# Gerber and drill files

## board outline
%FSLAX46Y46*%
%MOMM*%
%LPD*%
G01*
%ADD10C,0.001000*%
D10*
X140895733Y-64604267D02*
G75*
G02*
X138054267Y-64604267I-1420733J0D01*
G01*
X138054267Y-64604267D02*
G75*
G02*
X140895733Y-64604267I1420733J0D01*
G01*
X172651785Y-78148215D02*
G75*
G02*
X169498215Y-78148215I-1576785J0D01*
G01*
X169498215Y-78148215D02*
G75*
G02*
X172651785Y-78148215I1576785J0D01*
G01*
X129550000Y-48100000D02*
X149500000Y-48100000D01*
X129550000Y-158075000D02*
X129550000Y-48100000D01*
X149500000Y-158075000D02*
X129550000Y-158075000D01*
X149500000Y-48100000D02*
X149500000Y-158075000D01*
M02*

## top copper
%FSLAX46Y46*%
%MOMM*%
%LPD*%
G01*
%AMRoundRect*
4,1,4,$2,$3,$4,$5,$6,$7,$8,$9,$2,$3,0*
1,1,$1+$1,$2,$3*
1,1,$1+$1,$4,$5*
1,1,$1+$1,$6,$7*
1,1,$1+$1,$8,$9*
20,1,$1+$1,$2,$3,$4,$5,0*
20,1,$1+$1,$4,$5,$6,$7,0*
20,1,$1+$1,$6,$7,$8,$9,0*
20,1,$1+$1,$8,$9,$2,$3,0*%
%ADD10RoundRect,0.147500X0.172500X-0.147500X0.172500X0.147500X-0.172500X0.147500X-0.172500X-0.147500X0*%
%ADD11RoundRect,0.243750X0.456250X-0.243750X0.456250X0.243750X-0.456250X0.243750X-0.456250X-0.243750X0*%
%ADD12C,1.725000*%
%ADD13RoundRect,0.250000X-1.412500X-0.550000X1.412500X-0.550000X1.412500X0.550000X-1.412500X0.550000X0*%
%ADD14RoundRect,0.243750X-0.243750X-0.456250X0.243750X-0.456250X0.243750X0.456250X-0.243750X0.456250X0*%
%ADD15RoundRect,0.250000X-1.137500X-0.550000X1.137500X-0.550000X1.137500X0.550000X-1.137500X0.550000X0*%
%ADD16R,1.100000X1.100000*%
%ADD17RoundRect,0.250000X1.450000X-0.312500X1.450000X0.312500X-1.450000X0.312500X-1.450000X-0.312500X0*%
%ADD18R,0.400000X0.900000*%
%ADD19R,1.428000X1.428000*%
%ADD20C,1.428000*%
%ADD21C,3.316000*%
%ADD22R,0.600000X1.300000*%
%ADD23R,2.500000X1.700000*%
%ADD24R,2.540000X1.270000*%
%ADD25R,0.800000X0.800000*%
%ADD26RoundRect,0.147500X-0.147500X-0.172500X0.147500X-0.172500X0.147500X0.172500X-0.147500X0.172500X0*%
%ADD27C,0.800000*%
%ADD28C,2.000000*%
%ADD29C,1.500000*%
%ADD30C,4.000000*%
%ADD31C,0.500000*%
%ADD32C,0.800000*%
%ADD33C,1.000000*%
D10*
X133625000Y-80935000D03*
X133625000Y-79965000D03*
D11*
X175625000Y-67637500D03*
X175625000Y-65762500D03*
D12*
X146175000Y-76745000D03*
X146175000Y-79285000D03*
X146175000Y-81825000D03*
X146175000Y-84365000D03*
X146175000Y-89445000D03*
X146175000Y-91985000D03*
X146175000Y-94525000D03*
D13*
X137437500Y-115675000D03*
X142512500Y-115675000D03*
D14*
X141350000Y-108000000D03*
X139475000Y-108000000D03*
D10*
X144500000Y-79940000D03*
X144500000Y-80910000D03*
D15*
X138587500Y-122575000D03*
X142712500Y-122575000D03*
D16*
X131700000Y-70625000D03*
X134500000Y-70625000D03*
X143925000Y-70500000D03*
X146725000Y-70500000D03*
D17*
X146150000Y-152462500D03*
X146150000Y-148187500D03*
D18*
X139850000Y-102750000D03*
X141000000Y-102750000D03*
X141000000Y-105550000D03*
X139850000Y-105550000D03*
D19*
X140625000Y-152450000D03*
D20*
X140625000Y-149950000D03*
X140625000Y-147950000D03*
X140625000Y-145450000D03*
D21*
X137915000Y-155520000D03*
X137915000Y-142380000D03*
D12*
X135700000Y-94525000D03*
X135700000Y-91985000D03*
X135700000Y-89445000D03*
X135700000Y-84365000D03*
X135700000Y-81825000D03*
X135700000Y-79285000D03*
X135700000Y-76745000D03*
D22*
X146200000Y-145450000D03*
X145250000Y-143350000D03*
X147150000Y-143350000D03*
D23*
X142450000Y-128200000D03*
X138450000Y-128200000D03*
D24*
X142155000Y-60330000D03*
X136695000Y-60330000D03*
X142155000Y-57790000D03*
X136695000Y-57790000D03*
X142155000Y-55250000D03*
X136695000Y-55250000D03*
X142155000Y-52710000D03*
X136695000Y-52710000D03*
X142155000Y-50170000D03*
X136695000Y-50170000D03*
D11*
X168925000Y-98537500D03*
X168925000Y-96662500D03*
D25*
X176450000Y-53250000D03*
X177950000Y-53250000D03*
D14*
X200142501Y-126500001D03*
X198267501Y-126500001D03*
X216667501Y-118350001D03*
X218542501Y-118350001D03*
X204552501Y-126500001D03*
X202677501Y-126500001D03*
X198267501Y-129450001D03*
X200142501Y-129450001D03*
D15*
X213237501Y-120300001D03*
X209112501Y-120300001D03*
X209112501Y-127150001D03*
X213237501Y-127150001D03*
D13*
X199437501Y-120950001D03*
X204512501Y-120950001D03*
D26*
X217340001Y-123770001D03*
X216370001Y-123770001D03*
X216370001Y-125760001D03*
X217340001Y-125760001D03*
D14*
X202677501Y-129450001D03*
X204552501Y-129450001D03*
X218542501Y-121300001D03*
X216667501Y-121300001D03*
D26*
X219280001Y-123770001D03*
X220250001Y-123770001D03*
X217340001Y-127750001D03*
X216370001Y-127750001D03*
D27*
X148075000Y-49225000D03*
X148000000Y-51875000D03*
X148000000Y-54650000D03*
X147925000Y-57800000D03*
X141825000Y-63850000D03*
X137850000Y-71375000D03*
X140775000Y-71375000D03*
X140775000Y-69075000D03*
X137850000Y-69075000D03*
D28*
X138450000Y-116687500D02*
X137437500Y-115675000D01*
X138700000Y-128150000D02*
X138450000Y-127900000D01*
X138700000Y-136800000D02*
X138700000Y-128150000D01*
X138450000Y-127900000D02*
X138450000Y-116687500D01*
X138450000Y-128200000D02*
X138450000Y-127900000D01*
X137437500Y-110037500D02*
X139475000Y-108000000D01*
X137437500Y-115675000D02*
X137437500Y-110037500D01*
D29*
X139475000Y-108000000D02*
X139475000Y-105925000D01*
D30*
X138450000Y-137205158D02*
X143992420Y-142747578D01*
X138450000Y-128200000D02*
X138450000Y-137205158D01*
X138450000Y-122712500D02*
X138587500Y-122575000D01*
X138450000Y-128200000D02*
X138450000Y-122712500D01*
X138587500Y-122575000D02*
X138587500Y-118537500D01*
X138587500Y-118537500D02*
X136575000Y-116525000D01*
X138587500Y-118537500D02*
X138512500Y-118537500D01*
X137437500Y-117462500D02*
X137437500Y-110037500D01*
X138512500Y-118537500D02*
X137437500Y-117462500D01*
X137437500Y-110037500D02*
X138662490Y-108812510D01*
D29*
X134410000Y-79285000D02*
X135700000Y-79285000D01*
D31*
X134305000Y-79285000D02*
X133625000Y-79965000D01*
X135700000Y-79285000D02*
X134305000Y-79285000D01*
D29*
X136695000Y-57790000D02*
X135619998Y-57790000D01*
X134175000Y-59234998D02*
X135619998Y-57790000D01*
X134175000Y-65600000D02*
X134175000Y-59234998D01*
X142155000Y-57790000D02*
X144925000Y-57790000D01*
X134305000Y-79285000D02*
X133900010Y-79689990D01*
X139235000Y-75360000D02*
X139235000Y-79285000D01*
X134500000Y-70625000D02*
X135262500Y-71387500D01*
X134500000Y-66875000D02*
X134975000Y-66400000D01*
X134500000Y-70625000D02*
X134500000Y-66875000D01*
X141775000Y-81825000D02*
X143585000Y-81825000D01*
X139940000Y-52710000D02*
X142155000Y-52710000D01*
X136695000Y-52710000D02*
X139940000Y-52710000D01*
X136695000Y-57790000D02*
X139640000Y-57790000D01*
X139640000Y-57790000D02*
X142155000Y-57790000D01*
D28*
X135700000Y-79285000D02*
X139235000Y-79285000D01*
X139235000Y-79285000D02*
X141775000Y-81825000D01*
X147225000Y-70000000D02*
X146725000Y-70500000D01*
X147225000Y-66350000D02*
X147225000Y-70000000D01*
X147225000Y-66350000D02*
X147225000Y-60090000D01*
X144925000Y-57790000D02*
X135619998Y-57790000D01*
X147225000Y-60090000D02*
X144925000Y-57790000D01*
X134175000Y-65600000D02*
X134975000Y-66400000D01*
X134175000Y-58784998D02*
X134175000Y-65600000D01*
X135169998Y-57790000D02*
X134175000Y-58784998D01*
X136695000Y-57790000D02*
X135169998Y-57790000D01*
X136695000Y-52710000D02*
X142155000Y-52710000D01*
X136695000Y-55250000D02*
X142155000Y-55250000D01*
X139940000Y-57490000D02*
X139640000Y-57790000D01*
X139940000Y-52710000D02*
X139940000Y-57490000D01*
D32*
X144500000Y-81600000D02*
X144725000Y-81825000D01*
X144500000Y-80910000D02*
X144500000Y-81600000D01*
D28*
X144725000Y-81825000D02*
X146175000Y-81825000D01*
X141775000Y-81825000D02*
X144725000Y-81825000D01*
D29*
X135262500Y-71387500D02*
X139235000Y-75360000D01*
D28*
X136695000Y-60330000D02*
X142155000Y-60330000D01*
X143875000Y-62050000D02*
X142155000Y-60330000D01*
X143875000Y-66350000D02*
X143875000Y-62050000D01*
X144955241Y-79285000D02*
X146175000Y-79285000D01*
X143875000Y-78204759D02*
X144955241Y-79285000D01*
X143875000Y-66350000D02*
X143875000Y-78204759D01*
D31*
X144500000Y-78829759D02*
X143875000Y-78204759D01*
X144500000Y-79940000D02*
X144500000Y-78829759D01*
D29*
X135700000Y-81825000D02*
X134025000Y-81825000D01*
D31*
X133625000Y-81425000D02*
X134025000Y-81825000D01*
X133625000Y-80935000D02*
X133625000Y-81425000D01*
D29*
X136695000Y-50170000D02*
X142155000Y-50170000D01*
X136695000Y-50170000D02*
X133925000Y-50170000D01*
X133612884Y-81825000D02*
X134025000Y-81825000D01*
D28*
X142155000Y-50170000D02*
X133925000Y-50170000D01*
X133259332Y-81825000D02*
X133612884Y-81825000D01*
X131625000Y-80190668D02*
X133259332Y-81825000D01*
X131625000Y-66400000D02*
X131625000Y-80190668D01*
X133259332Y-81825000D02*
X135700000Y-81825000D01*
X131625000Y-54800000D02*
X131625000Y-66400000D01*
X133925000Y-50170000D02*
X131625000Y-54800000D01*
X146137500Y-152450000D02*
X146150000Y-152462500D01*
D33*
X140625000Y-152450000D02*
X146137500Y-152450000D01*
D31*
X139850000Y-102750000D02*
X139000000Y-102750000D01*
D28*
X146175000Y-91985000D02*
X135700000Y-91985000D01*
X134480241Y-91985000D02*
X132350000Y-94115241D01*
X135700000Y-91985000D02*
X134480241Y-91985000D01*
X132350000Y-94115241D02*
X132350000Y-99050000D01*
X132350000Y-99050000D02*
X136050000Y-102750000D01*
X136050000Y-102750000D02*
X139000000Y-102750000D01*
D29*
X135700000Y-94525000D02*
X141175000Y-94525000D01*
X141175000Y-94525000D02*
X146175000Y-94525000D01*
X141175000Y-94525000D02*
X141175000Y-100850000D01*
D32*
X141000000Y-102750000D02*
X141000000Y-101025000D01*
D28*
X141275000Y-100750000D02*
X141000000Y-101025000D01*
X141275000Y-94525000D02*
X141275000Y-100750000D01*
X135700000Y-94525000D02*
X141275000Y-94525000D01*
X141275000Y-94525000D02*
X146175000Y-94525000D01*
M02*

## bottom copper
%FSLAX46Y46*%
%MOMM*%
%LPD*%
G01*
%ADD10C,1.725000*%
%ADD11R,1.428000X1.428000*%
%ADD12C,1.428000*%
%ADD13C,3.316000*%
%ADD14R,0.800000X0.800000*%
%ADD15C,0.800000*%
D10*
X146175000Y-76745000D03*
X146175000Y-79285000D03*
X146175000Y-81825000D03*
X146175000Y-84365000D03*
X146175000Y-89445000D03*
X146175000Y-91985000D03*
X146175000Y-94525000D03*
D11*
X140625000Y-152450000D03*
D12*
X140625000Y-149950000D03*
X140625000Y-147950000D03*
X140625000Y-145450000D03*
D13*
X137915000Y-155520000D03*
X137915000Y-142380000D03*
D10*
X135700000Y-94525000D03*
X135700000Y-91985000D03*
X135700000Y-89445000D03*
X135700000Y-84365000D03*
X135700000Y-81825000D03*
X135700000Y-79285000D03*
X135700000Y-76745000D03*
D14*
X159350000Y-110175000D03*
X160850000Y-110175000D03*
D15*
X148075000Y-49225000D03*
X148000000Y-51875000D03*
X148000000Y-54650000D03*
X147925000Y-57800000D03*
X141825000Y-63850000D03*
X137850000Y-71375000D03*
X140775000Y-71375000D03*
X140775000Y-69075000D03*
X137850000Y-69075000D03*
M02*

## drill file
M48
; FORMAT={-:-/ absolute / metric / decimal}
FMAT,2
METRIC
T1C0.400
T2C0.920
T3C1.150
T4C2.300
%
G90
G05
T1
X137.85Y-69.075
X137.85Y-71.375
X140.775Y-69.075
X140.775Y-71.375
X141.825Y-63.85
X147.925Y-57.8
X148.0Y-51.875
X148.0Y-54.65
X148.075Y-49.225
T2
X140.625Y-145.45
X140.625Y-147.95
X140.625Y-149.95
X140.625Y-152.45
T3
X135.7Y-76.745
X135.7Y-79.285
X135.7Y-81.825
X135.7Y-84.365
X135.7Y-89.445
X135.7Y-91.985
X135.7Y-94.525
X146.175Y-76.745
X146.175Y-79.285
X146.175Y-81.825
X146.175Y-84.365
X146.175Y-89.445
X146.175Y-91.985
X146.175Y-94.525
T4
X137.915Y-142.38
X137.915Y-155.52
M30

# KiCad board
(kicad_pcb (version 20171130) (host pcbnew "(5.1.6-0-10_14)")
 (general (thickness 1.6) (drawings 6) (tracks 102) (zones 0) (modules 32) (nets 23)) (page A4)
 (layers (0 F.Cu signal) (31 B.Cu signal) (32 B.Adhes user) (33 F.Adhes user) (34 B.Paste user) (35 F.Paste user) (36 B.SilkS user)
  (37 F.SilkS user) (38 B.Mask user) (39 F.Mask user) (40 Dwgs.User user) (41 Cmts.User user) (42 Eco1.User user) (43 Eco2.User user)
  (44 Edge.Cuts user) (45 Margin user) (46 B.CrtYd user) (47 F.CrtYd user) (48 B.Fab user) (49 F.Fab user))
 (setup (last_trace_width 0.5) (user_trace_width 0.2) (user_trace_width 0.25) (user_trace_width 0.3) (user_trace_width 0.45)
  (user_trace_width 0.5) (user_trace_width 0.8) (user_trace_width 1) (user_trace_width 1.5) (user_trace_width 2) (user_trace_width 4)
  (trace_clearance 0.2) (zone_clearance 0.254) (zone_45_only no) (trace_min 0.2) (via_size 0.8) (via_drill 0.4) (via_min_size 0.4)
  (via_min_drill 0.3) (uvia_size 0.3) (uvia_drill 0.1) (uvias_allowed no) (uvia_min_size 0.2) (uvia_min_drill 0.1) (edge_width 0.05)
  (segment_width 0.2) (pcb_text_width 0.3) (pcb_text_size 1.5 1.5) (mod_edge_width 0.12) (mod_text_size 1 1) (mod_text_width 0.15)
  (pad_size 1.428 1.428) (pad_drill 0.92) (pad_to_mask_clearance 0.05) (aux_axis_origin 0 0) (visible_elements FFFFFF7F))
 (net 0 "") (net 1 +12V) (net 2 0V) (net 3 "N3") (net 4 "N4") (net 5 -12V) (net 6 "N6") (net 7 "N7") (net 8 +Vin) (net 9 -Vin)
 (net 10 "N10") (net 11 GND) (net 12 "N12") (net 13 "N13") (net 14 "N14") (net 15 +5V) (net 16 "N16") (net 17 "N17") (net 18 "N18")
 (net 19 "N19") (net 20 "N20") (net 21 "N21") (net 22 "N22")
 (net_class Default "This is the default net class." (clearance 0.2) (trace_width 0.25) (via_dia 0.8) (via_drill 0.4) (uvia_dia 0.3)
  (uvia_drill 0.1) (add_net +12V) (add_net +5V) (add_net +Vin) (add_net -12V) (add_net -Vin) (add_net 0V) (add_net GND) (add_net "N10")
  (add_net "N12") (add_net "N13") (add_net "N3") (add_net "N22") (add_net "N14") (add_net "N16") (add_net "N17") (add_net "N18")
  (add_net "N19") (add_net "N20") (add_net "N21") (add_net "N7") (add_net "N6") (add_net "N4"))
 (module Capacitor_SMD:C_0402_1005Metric (layer F.Cu) (at 133.625 80.45 90)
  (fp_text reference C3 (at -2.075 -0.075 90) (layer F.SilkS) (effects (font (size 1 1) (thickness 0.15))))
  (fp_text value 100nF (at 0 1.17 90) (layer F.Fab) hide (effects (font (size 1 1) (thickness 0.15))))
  (pad 1 smd roundrect (at -0.485 0 90) (size 0.59 0.64) (layers F.Cu F.Paste F.Mask) (roundrect_rratio 0.25) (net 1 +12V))
  (pad 2 smd roundrect (at 0.485 0 90) (size 0.59 0.64) (layers F.Cu F.Paste F.Mask) (roundrect_rratio 0.25) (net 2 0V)))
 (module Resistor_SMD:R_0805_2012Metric (layer F.Cu) (at 175.625 66.7 90)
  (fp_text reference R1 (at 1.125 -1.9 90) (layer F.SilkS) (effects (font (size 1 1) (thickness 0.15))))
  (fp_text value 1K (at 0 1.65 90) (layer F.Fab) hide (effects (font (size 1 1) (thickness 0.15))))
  (pad 1 smd roundrect (at -0.9375 0 90) (size 0.975 1.4) (layers F.Cu F.Paste F.Mask) (roundrect_rratio 0.25) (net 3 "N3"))
  (pad 2 smd roundrect (at 0.9375 0 90) (size 0.975 1.4) (layers F.Cu F.Paste F.Mask) (roundrect_rratio 0.25) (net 2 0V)))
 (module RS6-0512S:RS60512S (layer B.Cu) (at 146.175 94.525 90)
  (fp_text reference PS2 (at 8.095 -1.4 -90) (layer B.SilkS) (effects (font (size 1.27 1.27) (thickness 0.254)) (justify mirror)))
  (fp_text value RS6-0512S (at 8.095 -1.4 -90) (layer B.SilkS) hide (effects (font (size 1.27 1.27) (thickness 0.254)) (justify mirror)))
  (pad 8 thru_hole circle (at 17.78 0) (size 1.725 1.725) (drill 1.15) (layers *.Cu *.Mask B.SilkS) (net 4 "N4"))
  (pad 7 thru_hole circle (at 15.24 0) (size 1.725 1.725) (drill 1.15) (layers *.Cu *.Mask B.SilkS) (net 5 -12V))
  (pad 6 thru_hole circle (at 12.7 0) (size 1.725 1.725) (drill 1.15) (layers *.Cu *.Mask B.SilkS) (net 2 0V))
  (pad 5 thru_hole circle (at 10.16 0) (size 1.725 1.725) (drill 1.15) (layers *.Cu *.Mask B.SilkS) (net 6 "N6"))
  (pad 3 thru_hole circle (at 5.08 0) (size 1.725 1.725) (drill 1.15) (layers *.Cu *.Mask B.SilkS) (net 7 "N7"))
  (pad 2 thru_hole circle (at 2.54 0) (size 1.725 1.725) (drill 1.15) (layers *.Cu *.Mask B.SilkS) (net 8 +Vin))
  (pad 1 thru_hole circle (at 0 0) (size 1.725 1.725) (drill 1.15) (layers *.Cu *.Mask B.SilkS) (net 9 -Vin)))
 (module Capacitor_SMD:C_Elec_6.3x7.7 (layer F.Cu) (at 139.975 115.675)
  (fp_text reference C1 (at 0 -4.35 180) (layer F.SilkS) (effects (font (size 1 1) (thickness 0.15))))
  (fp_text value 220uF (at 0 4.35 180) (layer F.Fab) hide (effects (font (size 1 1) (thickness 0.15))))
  (pad 1 smd roundrect (at -2.5375 0) (size 3.325 1.6) (layers F.Cu F.Paste F.Mask) (roundrect_rratio 0.15625) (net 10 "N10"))
  (pad 2 smd roundrect (at 2.5375 0) (size 3.325 1.6) (layers F.Cu F.Paste F.Mask) (roundrect_rratio 0.15625) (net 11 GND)))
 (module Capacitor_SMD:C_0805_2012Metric (layer F.Cu) (at 140.4125 108)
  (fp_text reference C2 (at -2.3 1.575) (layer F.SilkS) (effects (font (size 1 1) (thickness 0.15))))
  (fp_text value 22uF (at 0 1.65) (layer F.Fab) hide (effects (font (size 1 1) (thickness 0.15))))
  (pad 2 smd roundrect (at 0.9375 0) (size 0.975 1.4) (layers F.Cu F.Paste F.Mask) (roundrect_rratio 0.25) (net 11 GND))
  (pad 1 smd roundrect (at -0.9375 0) (size 0.975 1.4) (layers F.Cu F.Paste F.Mask) (roundrect_rratio 0.25) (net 10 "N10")))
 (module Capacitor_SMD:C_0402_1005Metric (layer F.Cu) (at 144.5 80.425 90)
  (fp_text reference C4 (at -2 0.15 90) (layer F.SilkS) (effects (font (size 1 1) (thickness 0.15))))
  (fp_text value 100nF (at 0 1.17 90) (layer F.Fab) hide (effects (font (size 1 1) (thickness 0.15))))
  (pad 2 smd roundrect (at 0.485 0 90) (size 0.59 0.64) (layers F.Cu F.Paste F.Mask) (roundrect_rratio 0.25) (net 5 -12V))
  (pad 1 smd roundrect (at -0.485 0 90) (size 0.59 0.64) (layers F.Cu F.Paste F.Mask) (roundrect_rratio 0.25) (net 2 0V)))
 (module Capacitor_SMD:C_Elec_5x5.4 (layer F.Cu) (at 140.65 122.575)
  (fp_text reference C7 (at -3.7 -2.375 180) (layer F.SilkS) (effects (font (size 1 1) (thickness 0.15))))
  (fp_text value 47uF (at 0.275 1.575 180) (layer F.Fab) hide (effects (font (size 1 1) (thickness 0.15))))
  (pad 1 smd roundrect (at -2.0625 0) (size 2.775 1.6) (layers F.Cu F.Paste F.Mask) (roundrect_rratio 0.15625) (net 10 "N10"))
  (pad 2 smd roundrect (at 2.0625 0) (size 2.775 1.6) (layers F.Cu F.Paste F.Mask) (roundrect_rratio 0.15625) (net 11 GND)))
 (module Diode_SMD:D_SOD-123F (layer F.Cu) (at 133.1 70.625)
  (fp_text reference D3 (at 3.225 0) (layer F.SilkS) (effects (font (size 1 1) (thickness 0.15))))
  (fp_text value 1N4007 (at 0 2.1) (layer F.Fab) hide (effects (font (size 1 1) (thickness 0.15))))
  (pad 1 smd rect (at -1.4 0) (size 1.1 1.1) (layers F.Cu F.Paste F.Mask) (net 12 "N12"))
  (pad 2 smd rect (at 1.4 0) (size 1.1 1.1) (layers F.Cu F.Paste F.Mask) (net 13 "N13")))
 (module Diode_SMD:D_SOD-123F (layer F.Cu) (at 145.325 70.5 180)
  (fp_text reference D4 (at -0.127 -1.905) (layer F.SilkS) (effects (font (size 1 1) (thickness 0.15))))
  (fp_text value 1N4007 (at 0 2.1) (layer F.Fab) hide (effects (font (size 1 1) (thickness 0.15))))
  (pad 2 smd rect (at 1.4 0 180) (size 1.1 1.1) (layers F.Cu F.Paste F.Mask) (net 5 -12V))
  (pad 1 smd rect (at -1.4 0 180) (size 1.1 1.1) (layers F.Cu F.Paste F.Mask) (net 13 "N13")))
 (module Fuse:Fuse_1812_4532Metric (layer F.Cu) (at 146.15 150.325 90)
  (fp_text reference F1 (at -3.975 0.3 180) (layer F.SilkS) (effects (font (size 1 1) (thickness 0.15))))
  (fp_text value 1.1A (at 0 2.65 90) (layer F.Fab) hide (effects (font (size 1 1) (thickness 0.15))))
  (pad 1 smd roundrect (at -2.1375 0 90) (size 1.125 3.4) (layers F.Cu F.Paste F.Mask) (roundrect_rratio 0.222222) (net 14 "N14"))
  (pad 2 smd roundrect (at 2.1375 0 90) (size 1.125 3.4) (layers F.Cu F.Paste F.Mask) (roundrect_rratio 0.222222) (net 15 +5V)))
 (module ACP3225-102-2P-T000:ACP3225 (layer F.Cu) (at 140.425 104.15 90)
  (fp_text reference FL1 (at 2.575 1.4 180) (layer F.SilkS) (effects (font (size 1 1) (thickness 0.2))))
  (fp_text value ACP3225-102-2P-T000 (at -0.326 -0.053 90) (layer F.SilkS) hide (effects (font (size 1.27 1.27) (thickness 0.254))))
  (pad 4 smd rect (at 1.4 -0.575 180) (size 0.4 0.9) (layers F.Cu F.Paste F.Mask) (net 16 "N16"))
  (pad 3 smd rect (at 1.4 0.575 180) (size 0.4 0.9) (layers F.Cu F.Paste F.Mask) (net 9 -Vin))
  (pad 2 smd rect (at -1.4 0.575 180) (size 0.4 0.9) (layers F.Cu F.Paste F.Mask) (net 11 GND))
  (pad 1 smd rect (at -1.4 -0.575 180) (size 0.4 0.9) (layers F.Cu F.Paste F.Mask) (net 10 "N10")))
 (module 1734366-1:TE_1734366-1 (layer B.Cu) (at 140.625 152.45 90)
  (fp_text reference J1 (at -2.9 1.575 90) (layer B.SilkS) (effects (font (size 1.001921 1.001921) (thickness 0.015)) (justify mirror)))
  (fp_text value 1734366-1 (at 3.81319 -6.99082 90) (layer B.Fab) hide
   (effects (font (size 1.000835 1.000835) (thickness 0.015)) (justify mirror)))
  (pad 1 thru_hole rect (at 0 0 90) (size 1.428 1.428) (drill 0.92) (layers *.Cu *.Mask) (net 14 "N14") (zone_connect 1))
  (pad 2 thru_hole circle (at 2.5 0 90) (size 1.428 1.428) (drill 0.92) (layers *.Cu *.Mask) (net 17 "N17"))
  (pad 3 thru_hole circle (at 4.5 0 90) (size 1.428 1.428) (drill 0.92) (layers *.Cu *.Mask) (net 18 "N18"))
  (pad 4 thru_hole circle (at 7 0 90) (size 1.428 1.428) (drill 0.92) (layers *.Cu *.Mask) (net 11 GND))
  (pad SH1 thru_hole circle (at -3.07 -2.71 90) (size 3.316 3.316) (drill 2.3) (layers *.Cu *.Mask) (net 11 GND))
  (pad SH2 thru_hole circle (at 10.07 -2.71 90) (size 3.316 3.316) (drill 2.3) (layers *.Cu *.Mask) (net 11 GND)))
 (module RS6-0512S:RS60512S (layer B.Cu) (at 135.7 94.525 90)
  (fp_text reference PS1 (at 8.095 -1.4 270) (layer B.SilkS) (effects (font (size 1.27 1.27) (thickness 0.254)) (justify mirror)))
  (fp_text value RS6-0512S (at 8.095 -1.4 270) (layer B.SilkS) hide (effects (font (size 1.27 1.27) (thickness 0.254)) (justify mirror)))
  (pad 1 thru_hole circle (at 0 0) (size 1.725 1.725) (drill 1.15) (layers *.Cu *.Mask B.SilkS) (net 9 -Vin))
  (pad 2 thru_hole circle (at 2.54 0) (size 1.725 1.725) (drill 1.15) (layers *.Cu *.Mask B.SilkS) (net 8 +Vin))
  (pad 3 thru_hole circle (at 5.08 0) (size 1.725 1.725) (drill 1.15) (layers *.Cu *.Mask B.SilkS) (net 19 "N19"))
  (pad 5 thru_hole circle (at 10.16 0) (size 1.725 1.725) (drill 1.15) (layers *.Cu *.Mask B.SilkS) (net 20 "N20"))
  (pad 6 thru_hole circle (at 12.7 0) (size 1.725 1.725) (drill 1.15) (layers *.Cu *.Mask B.SilkS) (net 1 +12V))
  (pad 7 thru_hole circle (at 15.24 0) (size 1.725 1.725) (drill 1.15) (layers *.Cu *.Mask B.SilkS) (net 2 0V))
  (pad 8 thru_hole circle (at 17.78 0) (size 1.725 1.725) (drill 1.15) (layers *.Cu *.Mask B.SilkS) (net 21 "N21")))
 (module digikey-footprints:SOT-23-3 (layer F.Cu) (at 146.2 144.4 270)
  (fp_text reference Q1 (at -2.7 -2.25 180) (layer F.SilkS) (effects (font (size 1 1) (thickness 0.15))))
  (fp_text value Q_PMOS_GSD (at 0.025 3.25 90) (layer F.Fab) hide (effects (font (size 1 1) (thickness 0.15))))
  (pad 3 smd rect (at 1.05 0 270) (size 1.3 0.6) (layers F.Cu F.Paste F.Mask) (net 15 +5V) (solder_mask_margin 0.07))
  (pad 2 smd rect (at -1.05 0.95 270) (size 1.3 0.6) (layers F.Cu F.Paste F.Mask) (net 10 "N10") (solder_mask_margin 0.07))
  (pad 1 smd rect (at -1.05 -0.95 270) (size 1.3 0.6) (layers F.Cu F.Paste F.Mask) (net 11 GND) (solder_mask_margin 0.07)))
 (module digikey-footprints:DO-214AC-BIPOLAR (layer F.Cu) (at 140.45 128.2 180)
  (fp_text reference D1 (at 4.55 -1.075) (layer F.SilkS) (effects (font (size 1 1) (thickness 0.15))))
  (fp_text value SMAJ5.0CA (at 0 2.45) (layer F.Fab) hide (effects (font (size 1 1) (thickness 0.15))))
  (pad 2 smd rect (at -2 0 180) (size 2.5 1.7) (layers F.Cu F.Paste F.Mask) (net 11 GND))
  (pad 1 smd rect (at 2 0 180) (size 2.5 1.7) (layers F.Cu F.Paste F.Mask) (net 10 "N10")))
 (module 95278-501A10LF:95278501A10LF (layer F.Cu) (at 139.425 55.25 270)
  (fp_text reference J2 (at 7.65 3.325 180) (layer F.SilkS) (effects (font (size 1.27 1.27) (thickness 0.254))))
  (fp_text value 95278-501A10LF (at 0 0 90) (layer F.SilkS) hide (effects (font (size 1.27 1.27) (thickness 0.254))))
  (pad 10 smd rect (at 5.08 -2.73 270) (size 1.27 2.54) (layers F.Cu F.Paste F.Mask) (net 5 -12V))
  (pad 9 smd rect (at 5.08 2.73 270) (size 1.27 2.54) (layers F.Cu F.Paste F.Mask) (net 5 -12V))
  (pad 8 smd rect (at 2.54 -2.73 270) (size 1.27 2.54) (layers F.Cu F.Paste F.Mask) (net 13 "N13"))
  (pad 7 smd rect (at 2.54 2.73 270) (size 1.27 2.54) (layers F.Cu F.Paste F.Mask) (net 13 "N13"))
  (pad 6 smd rect (at 0 -2.73 270) (size 1.27 2.54) (layers F.Cu F.Paste F.Mask) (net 13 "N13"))
  (pad 5 smd rect (at 0 2.73 270) (size 1.27 2.54) (layers F.Cu F.Paste F.Mask) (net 13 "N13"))
  (pad 4 smd rect (at -2.54 -2.73 270) (size 1.27 2.54) (layers F.Cu F.Paste F.Mask) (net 13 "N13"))
  (pad 3 smd rect (at -2.54 2.73 270) (size 1.27 2.54) (layers F.Cu F.Paste F.Mask) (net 13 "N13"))
  (pad 2 smd rect (at -5.08 -2.73 270) (size 1.27 2.54) (layers F.Cu F.Paste F.Mask) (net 12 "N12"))
  (pad 1 smd rect (at -5.08 2.73 270) (size 1.27 2.54) (layers F.Cu F.Paste F.Mask) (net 12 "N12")))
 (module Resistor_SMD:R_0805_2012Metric (layer F.Cu) (at 168.925 97.6 90)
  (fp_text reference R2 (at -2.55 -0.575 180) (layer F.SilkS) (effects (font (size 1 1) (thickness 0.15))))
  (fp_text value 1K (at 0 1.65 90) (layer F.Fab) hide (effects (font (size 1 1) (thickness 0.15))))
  (pad 1 smd roundrect (at -0.9375 0 90) (size 0.975 1.4) (layers F.Cu F.Paste F.Mask) (roundrect_rratio 0.25) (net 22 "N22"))
  (pad 2 smd roundrect (at 0.9375 0 90) (size 0.975 1.4) (layers F.Cu F.Paste F.Mask) (roundrect_rratio 0.25) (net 5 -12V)))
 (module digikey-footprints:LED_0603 (layer F.Cu) (at 177.2 53.25)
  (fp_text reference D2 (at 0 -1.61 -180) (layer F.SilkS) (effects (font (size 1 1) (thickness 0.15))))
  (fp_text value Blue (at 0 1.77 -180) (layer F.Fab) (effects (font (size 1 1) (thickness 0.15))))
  (pad 1 smd rect (at -0.75 0) (size 0.8 0.8) (layers F.Cu F.Paste F.Mask) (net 3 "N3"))
  (pad 2 smd rect (at 0.75 0) (size 0.8 0.8) (layers F.Cu F.Paste F.Mask) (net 1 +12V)))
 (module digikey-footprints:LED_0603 (layer B.Cu) (at 160.1 110.175 180)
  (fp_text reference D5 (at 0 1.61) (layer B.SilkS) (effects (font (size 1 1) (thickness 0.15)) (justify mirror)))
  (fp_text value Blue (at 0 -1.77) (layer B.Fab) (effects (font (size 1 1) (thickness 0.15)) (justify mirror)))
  (pad 2 smd rect (at 0.75 0 180) (size 0.8 0.8) (layers B.Cu B.Paste B.Mask) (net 2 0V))
  (pad 1 smd rect (at -0.75 0 180) (size 0.8 0.8) (layers B.Cu B.Paste B.Mask) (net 22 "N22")))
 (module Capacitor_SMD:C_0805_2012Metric (layer F.Cu) (at 199.205001 126.500001)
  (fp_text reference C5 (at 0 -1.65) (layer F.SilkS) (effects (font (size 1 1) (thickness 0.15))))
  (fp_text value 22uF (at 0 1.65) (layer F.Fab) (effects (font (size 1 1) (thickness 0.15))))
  (pad 2 smd roundrect (at 0.9375 0) (size 0.975 1.4) (layers F.Cu F.Paste F.Mask) (roundrect_rratio 0.25) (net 2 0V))
  (pad 1 smd roundrect (at -0.9375 0) (size 0.975 1.4) (layers F.Cu F.Paste F.Mask) (roundrect_rratio 0.25) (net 1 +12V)))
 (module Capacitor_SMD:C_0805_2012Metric (layer F.Cu) (at 217.605001 118.350001)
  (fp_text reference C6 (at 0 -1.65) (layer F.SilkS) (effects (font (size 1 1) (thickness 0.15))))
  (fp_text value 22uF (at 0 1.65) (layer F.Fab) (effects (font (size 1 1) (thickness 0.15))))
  (pad 1 smd roundrect (at -0.9375 0) (size 0.975 1.4) (layers F.Cu F.Paste F.Mask) (roundrect_rratio 0.25) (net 2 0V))
  (pad 2 smd roundrect (at 0.9375 0) (size 0.975 1.4) (layers F.Cu F.Paste F.Mask) (roundrect_rratio 0.25) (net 5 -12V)))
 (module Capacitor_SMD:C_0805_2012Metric (layer F.Cu) (at 203.615001 126.500001)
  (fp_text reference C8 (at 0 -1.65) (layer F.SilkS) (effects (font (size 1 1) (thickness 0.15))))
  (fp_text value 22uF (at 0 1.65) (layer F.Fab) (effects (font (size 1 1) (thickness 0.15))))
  (pad 2 smd roundrect (at 0.9375 0) (size 0.975 1.4) (layers F.Cu F.Paste F.Mask) (roundrect_rratio 0.25) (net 2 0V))
  (pad 1 smd roundrect (at -0.9375 0) (size 0.975 1.4) (layers F.Cu F.Paste F.Mask) (roundrect_rratio 0.25) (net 1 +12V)))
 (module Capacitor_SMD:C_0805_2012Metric (layer F.Cu) (at 199.205001 129.450001)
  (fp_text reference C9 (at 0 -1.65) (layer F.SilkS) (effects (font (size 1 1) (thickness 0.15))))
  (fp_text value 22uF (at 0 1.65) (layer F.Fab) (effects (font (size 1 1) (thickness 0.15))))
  (pad 1 smd roundrect (at -0.9375 0) (size 0.975 1.4) (layers F.Cu F.Paste F.Mask) (roundrect_rratio 0.25) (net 2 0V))
  (pad 2 smd roundrect (at 0.9375 0) (size 0.975 1.4) (layers F.Cu F.Paste F.Mask) (roundrect_rratio 0.25) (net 5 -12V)))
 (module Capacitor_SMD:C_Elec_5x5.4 (layer F.Cu) (at 211.175001 120.300001)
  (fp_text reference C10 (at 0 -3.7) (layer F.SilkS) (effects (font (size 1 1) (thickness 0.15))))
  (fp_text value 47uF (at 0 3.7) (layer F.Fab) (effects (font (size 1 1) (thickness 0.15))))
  (pad 2 smd roundrect (at 2.0625 0) (size 2.775 1.6) (layers F.Cu F.Paste F.Mask) (roundrect_rratio 0.15625) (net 2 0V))
  (pad 1 smd roundrect (at -2.0625 0) (size 2.775 1.6) (layers F.Cu F.Paste F.Mask) (roundrect_rratio 0.15625) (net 1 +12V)))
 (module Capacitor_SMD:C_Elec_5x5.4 (layer F.Cu) (at 211.175001 127.150001)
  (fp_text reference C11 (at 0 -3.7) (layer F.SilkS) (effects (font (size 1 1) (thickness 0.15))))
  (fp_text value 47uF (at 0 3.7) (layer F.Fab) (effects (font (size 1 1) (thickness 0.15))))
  (pad 1 smd roundrect (at -2.0625 0) (size 2.775 1.6) (layers F.Cu F.Paste F.Mask) (roundrect_rratio 0.15625) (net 2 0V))
  (pad 2 smd roundrect (at 2.0625 0) (size 2.775 1.6) (layers F.Cu F.Paste F.Mask) (roundrect_rratio 0.15625) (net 5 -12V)))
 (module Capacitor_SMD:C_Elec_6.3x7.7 (layer F.Cu) (at 201.975001 120.950001)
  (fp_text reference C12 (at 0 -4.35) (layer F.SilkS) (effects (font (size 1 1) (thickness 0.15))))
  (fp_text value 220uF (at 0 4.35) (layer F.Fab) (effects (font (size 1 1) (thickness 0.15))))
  (pad 1 smd roundrect (at -2.5375 0) (size 3.325 1.6) (layers F.Cu F.Paste F.Mask) (roundrect_rratio 0.15625) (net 10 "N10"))
  (pad 2 smd roundrect (at 2.5375 0) (size 3.325 1.6) (layers F.Cu F.Paste F.Mask) (roundrect_rratio 0.15625) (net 11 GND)))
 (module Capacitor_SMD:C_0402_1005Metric (layer F.Cu) (at 216.855001 123.770001)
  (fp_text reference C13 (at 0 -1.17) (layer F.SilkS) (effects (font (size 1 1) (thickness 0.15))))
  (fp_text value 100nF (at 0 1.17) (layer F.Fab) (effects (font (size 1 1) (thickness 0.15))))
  (pad 2 smd roundrect (at 0.485 0) (size 0.59 0.64) (layers F.Cu F.Paste F.Mask) (roundrect_rratio 0.25) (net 13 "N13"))
  (pad 1 smd roundrect (at -0.485 0) (size 0.59 0.64) (layers F.Cu F.Paste F.Mask) (roundrect_rratio 0.25) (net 12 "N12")))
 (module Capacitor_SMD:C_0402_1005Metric (layer F.Cu) (at 216.855001 125.760001)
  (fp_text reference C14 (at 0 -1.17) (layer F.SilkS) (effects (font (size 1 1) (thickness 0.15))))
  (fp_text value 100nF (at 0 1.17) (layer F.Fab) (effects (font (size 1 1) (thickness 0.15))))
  (pad 1 smd roundrect (at -0.485 0) (size 0.59 0.64) (layers F.Cu F.Paste F.Mask) (roundrect_rratio 0.25) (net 13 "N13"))
  (pad 2 smd roundrect (at 0.485 0) (size 0.59 0.64) (layers F.Cu F.Paste F.Mask) (roundrect_rratio 0.25) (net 5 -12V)))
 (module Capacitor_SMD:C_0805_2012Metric (layer F.Cu) (at 203.615001 129.450001)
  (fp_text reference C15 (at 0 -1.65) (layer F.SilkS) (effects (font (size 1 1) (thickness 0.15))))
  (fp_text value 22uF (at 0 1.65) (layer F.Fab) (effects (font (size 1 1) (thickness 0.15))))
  (pad 1 smd roundrect (at -0.9375 0) (size 0.975 1.4) (layers F.Cu F.Paste F.Mask) (roundrect_rratio 0.25) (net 8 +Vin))
  (pad 2 smd roundrect (at 0.9375 0) (size 0.975 1.4) (layers F.Cu F.Paste F.Mask) (roundrect_rratio 0.25) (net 9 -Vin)))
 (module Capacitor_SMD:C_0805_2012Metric (layer F.Cu) (at 217.605001 121.300001)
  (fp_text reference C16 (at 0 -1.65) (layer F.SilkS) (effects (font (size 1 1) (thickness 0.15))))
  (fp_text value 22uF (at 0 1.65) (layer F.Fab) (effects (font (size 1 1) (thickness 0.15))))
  (pad 2 smd roundrect (at 0.9375 0) (size 0.975 1.4) (layers F.Cu F.Paste F.Mask) (roundrect_rratio 0.25) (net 9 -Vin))
  (pad 1 smd roundrect (at -0.9375 0) (size 0.975 1.4) (layers F.Cu F.Paste F.Mask) (roundrect_rratio 0.25) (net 8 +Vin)))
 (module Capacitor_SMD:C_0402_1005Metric (layer F.Cu) (at 219.765001 123.770001)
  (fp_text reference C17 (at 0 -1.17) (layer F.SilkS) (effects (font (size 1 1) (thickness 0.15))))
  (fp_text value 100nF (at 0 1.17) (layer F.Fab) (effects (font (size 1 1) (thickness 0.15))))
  (pad 1 smd roundrect (at -0.485 0) (size 0.59 0.64) (layers F.Cu F.Paste F.Mask) (roundrect_rratio 0.25) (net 8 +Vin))
  (pad 2 smd roundrect (at 0.485 0) (size 0.59 0.64) (layers F.Cu F.Paste F.Mask) (roundrect_rratio 0.25) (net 9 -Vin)))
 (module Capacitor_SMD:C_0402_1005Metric (layer F.Cu) (at 216.855001 127.750001)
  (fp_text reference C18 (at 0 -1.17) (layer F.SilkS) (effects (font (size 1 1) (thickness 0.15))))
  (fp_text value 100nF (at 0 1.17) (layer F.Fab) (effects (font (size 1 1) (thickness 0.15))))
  (pad 2 smd roundrect (at 0.485 0) (size 0.59 0.64) (layers F.Cu F.Paste F.Mask) (roundrect_rratio 0.25) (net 9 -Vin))
  (pad 1 smd roundrect (at -0.485 0) (size 0.59 0.64) (layers F.Cu F.Paste F.Mask) (roundrect_rratio 0.25) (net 8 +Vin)))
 (gr_circle (center 139.475 64.604267) (end 140.895733 64.604267) (layer Edge.Cuts) (width 0.001))
 (gr_circle (center 171.075 78.148215) (end 172.651785 78.148215) (layer Edge.Cuts) (width 0.001))
 (gr_line (start 129.55 48.1) (end 149.5 48.1) (layer Edge.Cuts) (width 0.001))
 (gr_line (start 129.55 158.075) (end 129.55 48.1) (layer Edge.Cuts) (width 0.001))
 (gr_line (start 149.5 158.075) (end 129.55 158.075) (layer Edge.Cuts) (width 0.001))
 (gr_line (start 149.5 48.1) (end 149.5 158.075) (layer Edge.Cuts) (width 0.001))
 (segment (start 138.45 116.6875) (end 137.4375 115.675) (width 2) (layer F.Cu) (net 10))
 (segment (start 138.7 128.15) (end 138.45 127.9) (width 2) (layer F.Cu) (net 10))
 (segment (start 138.7 136.8) (end 138.7 128.15) (width 2) (layer F.Cu) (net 10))
 (segment (start 138.45 127.9) (end 138.45 116.6875) (width 2) (layer F.Cu) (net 10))
 (segment (start 138.45 128.2) (end 138.45 127.9) (width 2) (layer F.Cu) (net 10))
 (segment (start 137.4375 110.0375) (end 139.475 108) (width 2) (layer F.Cu) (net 10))
 (segment (start 137.4375 115.675) (end 137.4375 110.0375) (width 2) (layer F.Cu) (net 10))
 (segment (start 139.475 108) (end 139.475 105.925) (width 1.5) (layer F.Cu) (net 10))
 (segment (start 138.45 137.205158) (end 143.99242 142.747578) (width 4) (layer F.Cu) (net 10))
 (segment (start 138.45 128.2) (end 138.45 137.205158) (width 4) (layer F.Cu) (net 10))
 (segment (start 138.45 122.7125) (end 138.5875 122.575) (width 4) (layer F.Cu) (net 10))
 (segment (start 138.45 128.2) (end 138.45 122.7125) (width 4) (layer F.Cu) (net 10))
 (segment (start 138.5875 122.575) (end 138.5875 118.5375) (width 4) (layer F.Cu) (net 10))
 (segment (start 138.5875 118.5375) (end 136.575 116.525) (width 4) (layer F.Cu) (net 10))
 (segment (start 138.5875 118.5375) (end 138.5125 118.5375) (width 4) (layer F.Cu) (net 10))
 (segment (start 137.4375 117.4625) (end 137.4375 110.0375) (width 4) (layer F.Cu) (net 10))
 (segment (start 138.5125 118.5375) (end 137.4375 117.4625) (width 4) (layer F.Cu) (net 10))
 (segment (start 137.4375 110.0375) (end 138.66249 108.81251) (width 4) (layer F.Cu) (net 10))
 (segment (start 134.41 79.285) (end 135.7 79.285) (width 1.5) (layer F.Cu) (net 2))
 (segment (start 134.305 79.285) (end 133.625 79.965) (width 0.5) (layer F.Cu) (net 2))
 (segment (start 135.7 79.285) (end 134.305 79.285) (width 0.5) (layer F.Cu) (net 2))
 (segment (start 136.695 57.79) (end 135.619998 57.79) (width 1.5) (layer F.Cu) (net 2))
 (segment (start 134.175 59.234998) (end 135.619998 57.79) (width 1.5) (layer F.Cu) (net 2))
 (segment (start 134.175 65.6) (end 134.175 59.234998) (width 1.5) (layer F.Cu) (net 2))
 (segment (start 142.155 57.79) (end 144.925 57.79) (width 1.5) (layer F.Cu) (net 2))
 (segment (start 134.305 79.285) (end 133.90001 79.68999) (width 1.5) (layer F.Cu) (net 2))
 (segment (start 139.235 75.36) (end 139.235 79.285) (width 1.5) (layer F.Cu) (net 2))
 (segment (start 134.5 70.625) (end 135.2625 71.3875) (width 1.5) (layer F.Cu) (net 2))
 (segment (start 134.5 66.875) (end 134.975 66.4) (width 1.5) (layer F.Cu) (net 2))
 (segment (start 134.5 70.625) (end 134.5 66.875) (width 1.5) (layer F.Cu) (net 2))
 (segment (start 141.775 81.825) (end 143.585 81.825) (width 1.5) (layer F.Cu) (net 2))
 (segment (start 139.94 52.71) (end 142.155 52.71) (width 1.5) (layer F.Cu) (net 2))
 (segment (start 136.695 52.71) (end 139.94 52.71) (width 1.5) (layer F.Cu) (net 2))
 (segment (start 136.695 57.79) (end 139.64 57.79) (width 1.5) (layer F.Cu) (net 2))
 (segment (start 139.64 57.79) (end 142.155 57.79) (width 1.5) (layer F.Cu) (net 2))
 (segment (start 135.7 79.285) (end 139.235 79.285) (width 2) (layer F.Cu) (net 2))
 (segment (start 139.235 79.285) (end 141.775 81.825) (width 2) (layer F.Cu) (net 2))
 (segment (start 147.225 70) (end 146.725 70.5) (width 2) (layer F.Cu) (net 2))
 (segment (start 147.225 66.35) (end 147.225 70) (width 2) (layer F.Cu) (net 2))
 (segment (start 147.225 66.35) (end 147.225 60.09) (width 2) (layer F.Cu) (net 2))
 (segment (start 144.925 57.79) (end 135.619998 57.79) (width 2) (layer F.Cu) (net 2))
 (segment (start 147.225 60.09) (end 144.925 57.79) (width 2) (layer F.Cu) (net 2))
 (segment (start 134.175 65.6) (end 134.975 66.4) (width 2) (layer F.Cu) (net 2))
 (segment (start 134.175 58.784998) (end 134.175 65.6) (width 2) (layer F.Cu) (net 2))
 (segment (start 135.169998 57.79) (end 134.175 58.784998) (width 2) (layer F.Cu) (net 2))
 (segment (start 136.695 57.79) (end 135.169998 57.79) (width 2) (layer F.Cu) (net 2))
 (segment (start 136.695 52.71) (end 142.155 52.71) (width 2) (layer F.Cu) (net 2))
 (segment (start 136.695 55.25) (end 142.155 55.25) (width 2) (layer F.Cu) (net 13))
 (segment (start 139.94 57.49) (end 139.64 57.79) (width 2) (layer F.Cu) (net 2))
 (segment (start 139.94 52.71) (end 139.94 57.49) (width 2) (layer F.Cu) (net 2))
 (segment (start 144.5 81.6) (end 144.725 81.825) (width 0.8) (layer F.Cu) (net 2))
 (segment (start 144.5 80.91) (end 144.5 81.6) (width 0.8) (layer F.Cu) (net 2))
 (segment (start 144.725 81.825) (end 146.175 81.825) (width 2) (layer F.Cu) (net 2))
 (segment (start 141.775 81.825) (end 144.725 81.825) (width 2) (layer F.Cu) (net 2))
 (via (at 148.075 49.225) (size 0.8) (drill 0.4) (layers F.Cu B.Cu) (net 2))
 (via (at 148 51.875) (size 0.8) (drill 0.4) (layers F.Cu B.Cu) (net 2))
 (via (at 148 54.65) (size 0.8) (drill 0.4) (layers F.Cu B.Cu) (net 2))
 (via (at 147.925 57.8) (size 0.8) (drill 0.4) (layers F.Cu B.Cu) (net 2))
 (segment (start 135.2625 71.3875) (end 139.235 75.36) (width 1.5) (layer F.Cu) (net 2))
 (via (at 141.825 63.85) (size 0.8) (drill 0.4) (layers F.Cu B.Cu) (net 2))
 (via (at 137.85 71.375) (size 0.8) (drill 0.4) (layers F.Cu B.Cu) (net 2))
 (via (at 140.775 71.375) (size 0.8) (drill 0.4) (layers F.Cu B.Cu) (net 2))
 (via (at 140.775 69.075) (size 0.8) (drill 0.4) (layers F.Cu B.Cu) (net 2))
 (via (at 137.85 69.075) (size 0.8) (drill 0.4) (layers F.Cu B.Cu) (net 2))
 (segment (start 136.695 60.33) (end 142.155 60.33) (width 2) (layer F.Cu) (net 5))
 (segment (start 143.875 62.05) (end 142.155 60.33) (width 2) (layer F.Cu) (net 5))
 (segment (start 143.875 66.35) (end 143.875 62.05) (width 2) (layer F.Cu) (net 5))
 (segment (start 144.955241 79.285) (end 146.175 79.285) (width 2) (layer F.Cu) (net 5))
 (segment (start 143.875 78.204759) (end 144.955241 79.285) (width 2) (layer F.Cu) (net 5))
 (segment (start 143.875 66.35) (end 143.875 78.204759) (width 2) (layer F.Cu) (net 5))
 (segment (start 144.5 78.829759) (end 143.875 78.204759) (width 0.5) (layer F.Cu) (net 5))
 (segment (start 144.5 79.94) (end 144.5 78.829759) (width 0.5) (layer F.Cu) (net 5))
 (segment (start 135.7 81.825) (end 134.025 81.825) (width 1.5) (layer F.Cu) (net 1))
 (segment (start 133.625 81.425) (end 134.025 81.825) (width 0.5) (layer F.Cu) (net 1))
 (segment (start 133.625 80.935) (end 133.625 81.425) (width 0.5) (layer F.Cu) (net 1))
 (segment (start 136.695 50.17) (end 142.155 50.17) (width 1.5) (layer F.Cu) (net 1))
 (segment (start 136.695 50.17) (end 133.925 50.17) (width 1.5) (layer F.Cu) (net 1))
 (segment (start 133.612884 81.825) (end 134.025 81.825) (width 1.5) (layer F.Cu) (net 1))
 (segment (start 142.155 50.17) (end 133.925 50.17) (width 2) (layer F.Cu) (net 1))
 (segment (start 133.259332 81.825) (end 133.612884 81.825) (width 2) (layer F.Cu) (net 1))
 (segment (start 131.625 80.190668) (end 133.259332 81.825) (width 2) (layer F.Cu) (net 1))
 (segment (start 131.625 66.4) (end 131.625 80.190668) (width 2) (layer F.Cu) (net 1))
 (segment (start 133.259332 81.825) (end 135.7 81.825) (width 2) (layer F.Cu) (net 1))
 (segment (start 131.625 54.8) (end 131.625 66.4) (width 2) (layer F.Cu) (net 1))
 (segment (start 133.925 50.17) (end 131.625 54.8) (width 2) (layer F.Cu) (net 1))
 (segment (start 146.1375 152.45) (end 146.15 152.4625) (width 2) (layer F.Cu) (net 14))
 (segment (start 140.625 152.45) (end 146.1375 152.45) (width 1) (layer F.Cu) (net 14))
 (segment (start 139.85 102.75) (end 139 102.75) (width 0.5) (layer F.Cu) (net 8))
 (segment (start 146.175 91.985) (end 135.7 91.985) (width 2) (layer F.Cu) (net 8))
 (segment (start 134.480241 91.985) (end 132.35 94.115241) (width 2) (layer F.Cu) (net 8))
 (segment (start 135.7 91.985) (end 134.480241 91.985) (width 2) (layer F.Cu) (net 8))
 (segment (start 132.35 94.115241) (end 132.35 99.05) (width 2) (layer F.Cu) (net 8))
 (segment (start 132.35 99.05) (end 136.05 102.75) (width 2) (layer F.Cu) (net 8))
 (segment (start 136.05 102.75) (end 139 102.75) (width 2) (layer F.Cu) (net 8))
 (segment (start 135.7 94.525) (end 141.175 94.525) (width 1.5) (layer F.Cu) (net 9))
 (segment (start 141.175 94.525) (end 146.175 94.525) (width 1.5) (layer F.Cu) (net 9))
 (segment (start 141.175 94.525) (end 141.175 100.85) (width 1.5) (layer F.Cu) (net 9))
 (segment (start 141 102.75) (end 141 101.025) (width 0.8) (layer F.Cu) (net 9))
 (segment (start 141.275 100.75) (end 141 101.025) (width 2) (layer F.Cu) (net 9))
 (segment (start 141.275 94.525) (end 141.275 100.75) (width 2) (layer F.Cu) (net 9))
 (segment (start 135.7 94.525) (end 141.275 94.525) (width 2) (layer F.Cu) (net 9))
 (segment (start 141.275 94.525) (end 146.175 94.525) (width 2) (layer F.Cu) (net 9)))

